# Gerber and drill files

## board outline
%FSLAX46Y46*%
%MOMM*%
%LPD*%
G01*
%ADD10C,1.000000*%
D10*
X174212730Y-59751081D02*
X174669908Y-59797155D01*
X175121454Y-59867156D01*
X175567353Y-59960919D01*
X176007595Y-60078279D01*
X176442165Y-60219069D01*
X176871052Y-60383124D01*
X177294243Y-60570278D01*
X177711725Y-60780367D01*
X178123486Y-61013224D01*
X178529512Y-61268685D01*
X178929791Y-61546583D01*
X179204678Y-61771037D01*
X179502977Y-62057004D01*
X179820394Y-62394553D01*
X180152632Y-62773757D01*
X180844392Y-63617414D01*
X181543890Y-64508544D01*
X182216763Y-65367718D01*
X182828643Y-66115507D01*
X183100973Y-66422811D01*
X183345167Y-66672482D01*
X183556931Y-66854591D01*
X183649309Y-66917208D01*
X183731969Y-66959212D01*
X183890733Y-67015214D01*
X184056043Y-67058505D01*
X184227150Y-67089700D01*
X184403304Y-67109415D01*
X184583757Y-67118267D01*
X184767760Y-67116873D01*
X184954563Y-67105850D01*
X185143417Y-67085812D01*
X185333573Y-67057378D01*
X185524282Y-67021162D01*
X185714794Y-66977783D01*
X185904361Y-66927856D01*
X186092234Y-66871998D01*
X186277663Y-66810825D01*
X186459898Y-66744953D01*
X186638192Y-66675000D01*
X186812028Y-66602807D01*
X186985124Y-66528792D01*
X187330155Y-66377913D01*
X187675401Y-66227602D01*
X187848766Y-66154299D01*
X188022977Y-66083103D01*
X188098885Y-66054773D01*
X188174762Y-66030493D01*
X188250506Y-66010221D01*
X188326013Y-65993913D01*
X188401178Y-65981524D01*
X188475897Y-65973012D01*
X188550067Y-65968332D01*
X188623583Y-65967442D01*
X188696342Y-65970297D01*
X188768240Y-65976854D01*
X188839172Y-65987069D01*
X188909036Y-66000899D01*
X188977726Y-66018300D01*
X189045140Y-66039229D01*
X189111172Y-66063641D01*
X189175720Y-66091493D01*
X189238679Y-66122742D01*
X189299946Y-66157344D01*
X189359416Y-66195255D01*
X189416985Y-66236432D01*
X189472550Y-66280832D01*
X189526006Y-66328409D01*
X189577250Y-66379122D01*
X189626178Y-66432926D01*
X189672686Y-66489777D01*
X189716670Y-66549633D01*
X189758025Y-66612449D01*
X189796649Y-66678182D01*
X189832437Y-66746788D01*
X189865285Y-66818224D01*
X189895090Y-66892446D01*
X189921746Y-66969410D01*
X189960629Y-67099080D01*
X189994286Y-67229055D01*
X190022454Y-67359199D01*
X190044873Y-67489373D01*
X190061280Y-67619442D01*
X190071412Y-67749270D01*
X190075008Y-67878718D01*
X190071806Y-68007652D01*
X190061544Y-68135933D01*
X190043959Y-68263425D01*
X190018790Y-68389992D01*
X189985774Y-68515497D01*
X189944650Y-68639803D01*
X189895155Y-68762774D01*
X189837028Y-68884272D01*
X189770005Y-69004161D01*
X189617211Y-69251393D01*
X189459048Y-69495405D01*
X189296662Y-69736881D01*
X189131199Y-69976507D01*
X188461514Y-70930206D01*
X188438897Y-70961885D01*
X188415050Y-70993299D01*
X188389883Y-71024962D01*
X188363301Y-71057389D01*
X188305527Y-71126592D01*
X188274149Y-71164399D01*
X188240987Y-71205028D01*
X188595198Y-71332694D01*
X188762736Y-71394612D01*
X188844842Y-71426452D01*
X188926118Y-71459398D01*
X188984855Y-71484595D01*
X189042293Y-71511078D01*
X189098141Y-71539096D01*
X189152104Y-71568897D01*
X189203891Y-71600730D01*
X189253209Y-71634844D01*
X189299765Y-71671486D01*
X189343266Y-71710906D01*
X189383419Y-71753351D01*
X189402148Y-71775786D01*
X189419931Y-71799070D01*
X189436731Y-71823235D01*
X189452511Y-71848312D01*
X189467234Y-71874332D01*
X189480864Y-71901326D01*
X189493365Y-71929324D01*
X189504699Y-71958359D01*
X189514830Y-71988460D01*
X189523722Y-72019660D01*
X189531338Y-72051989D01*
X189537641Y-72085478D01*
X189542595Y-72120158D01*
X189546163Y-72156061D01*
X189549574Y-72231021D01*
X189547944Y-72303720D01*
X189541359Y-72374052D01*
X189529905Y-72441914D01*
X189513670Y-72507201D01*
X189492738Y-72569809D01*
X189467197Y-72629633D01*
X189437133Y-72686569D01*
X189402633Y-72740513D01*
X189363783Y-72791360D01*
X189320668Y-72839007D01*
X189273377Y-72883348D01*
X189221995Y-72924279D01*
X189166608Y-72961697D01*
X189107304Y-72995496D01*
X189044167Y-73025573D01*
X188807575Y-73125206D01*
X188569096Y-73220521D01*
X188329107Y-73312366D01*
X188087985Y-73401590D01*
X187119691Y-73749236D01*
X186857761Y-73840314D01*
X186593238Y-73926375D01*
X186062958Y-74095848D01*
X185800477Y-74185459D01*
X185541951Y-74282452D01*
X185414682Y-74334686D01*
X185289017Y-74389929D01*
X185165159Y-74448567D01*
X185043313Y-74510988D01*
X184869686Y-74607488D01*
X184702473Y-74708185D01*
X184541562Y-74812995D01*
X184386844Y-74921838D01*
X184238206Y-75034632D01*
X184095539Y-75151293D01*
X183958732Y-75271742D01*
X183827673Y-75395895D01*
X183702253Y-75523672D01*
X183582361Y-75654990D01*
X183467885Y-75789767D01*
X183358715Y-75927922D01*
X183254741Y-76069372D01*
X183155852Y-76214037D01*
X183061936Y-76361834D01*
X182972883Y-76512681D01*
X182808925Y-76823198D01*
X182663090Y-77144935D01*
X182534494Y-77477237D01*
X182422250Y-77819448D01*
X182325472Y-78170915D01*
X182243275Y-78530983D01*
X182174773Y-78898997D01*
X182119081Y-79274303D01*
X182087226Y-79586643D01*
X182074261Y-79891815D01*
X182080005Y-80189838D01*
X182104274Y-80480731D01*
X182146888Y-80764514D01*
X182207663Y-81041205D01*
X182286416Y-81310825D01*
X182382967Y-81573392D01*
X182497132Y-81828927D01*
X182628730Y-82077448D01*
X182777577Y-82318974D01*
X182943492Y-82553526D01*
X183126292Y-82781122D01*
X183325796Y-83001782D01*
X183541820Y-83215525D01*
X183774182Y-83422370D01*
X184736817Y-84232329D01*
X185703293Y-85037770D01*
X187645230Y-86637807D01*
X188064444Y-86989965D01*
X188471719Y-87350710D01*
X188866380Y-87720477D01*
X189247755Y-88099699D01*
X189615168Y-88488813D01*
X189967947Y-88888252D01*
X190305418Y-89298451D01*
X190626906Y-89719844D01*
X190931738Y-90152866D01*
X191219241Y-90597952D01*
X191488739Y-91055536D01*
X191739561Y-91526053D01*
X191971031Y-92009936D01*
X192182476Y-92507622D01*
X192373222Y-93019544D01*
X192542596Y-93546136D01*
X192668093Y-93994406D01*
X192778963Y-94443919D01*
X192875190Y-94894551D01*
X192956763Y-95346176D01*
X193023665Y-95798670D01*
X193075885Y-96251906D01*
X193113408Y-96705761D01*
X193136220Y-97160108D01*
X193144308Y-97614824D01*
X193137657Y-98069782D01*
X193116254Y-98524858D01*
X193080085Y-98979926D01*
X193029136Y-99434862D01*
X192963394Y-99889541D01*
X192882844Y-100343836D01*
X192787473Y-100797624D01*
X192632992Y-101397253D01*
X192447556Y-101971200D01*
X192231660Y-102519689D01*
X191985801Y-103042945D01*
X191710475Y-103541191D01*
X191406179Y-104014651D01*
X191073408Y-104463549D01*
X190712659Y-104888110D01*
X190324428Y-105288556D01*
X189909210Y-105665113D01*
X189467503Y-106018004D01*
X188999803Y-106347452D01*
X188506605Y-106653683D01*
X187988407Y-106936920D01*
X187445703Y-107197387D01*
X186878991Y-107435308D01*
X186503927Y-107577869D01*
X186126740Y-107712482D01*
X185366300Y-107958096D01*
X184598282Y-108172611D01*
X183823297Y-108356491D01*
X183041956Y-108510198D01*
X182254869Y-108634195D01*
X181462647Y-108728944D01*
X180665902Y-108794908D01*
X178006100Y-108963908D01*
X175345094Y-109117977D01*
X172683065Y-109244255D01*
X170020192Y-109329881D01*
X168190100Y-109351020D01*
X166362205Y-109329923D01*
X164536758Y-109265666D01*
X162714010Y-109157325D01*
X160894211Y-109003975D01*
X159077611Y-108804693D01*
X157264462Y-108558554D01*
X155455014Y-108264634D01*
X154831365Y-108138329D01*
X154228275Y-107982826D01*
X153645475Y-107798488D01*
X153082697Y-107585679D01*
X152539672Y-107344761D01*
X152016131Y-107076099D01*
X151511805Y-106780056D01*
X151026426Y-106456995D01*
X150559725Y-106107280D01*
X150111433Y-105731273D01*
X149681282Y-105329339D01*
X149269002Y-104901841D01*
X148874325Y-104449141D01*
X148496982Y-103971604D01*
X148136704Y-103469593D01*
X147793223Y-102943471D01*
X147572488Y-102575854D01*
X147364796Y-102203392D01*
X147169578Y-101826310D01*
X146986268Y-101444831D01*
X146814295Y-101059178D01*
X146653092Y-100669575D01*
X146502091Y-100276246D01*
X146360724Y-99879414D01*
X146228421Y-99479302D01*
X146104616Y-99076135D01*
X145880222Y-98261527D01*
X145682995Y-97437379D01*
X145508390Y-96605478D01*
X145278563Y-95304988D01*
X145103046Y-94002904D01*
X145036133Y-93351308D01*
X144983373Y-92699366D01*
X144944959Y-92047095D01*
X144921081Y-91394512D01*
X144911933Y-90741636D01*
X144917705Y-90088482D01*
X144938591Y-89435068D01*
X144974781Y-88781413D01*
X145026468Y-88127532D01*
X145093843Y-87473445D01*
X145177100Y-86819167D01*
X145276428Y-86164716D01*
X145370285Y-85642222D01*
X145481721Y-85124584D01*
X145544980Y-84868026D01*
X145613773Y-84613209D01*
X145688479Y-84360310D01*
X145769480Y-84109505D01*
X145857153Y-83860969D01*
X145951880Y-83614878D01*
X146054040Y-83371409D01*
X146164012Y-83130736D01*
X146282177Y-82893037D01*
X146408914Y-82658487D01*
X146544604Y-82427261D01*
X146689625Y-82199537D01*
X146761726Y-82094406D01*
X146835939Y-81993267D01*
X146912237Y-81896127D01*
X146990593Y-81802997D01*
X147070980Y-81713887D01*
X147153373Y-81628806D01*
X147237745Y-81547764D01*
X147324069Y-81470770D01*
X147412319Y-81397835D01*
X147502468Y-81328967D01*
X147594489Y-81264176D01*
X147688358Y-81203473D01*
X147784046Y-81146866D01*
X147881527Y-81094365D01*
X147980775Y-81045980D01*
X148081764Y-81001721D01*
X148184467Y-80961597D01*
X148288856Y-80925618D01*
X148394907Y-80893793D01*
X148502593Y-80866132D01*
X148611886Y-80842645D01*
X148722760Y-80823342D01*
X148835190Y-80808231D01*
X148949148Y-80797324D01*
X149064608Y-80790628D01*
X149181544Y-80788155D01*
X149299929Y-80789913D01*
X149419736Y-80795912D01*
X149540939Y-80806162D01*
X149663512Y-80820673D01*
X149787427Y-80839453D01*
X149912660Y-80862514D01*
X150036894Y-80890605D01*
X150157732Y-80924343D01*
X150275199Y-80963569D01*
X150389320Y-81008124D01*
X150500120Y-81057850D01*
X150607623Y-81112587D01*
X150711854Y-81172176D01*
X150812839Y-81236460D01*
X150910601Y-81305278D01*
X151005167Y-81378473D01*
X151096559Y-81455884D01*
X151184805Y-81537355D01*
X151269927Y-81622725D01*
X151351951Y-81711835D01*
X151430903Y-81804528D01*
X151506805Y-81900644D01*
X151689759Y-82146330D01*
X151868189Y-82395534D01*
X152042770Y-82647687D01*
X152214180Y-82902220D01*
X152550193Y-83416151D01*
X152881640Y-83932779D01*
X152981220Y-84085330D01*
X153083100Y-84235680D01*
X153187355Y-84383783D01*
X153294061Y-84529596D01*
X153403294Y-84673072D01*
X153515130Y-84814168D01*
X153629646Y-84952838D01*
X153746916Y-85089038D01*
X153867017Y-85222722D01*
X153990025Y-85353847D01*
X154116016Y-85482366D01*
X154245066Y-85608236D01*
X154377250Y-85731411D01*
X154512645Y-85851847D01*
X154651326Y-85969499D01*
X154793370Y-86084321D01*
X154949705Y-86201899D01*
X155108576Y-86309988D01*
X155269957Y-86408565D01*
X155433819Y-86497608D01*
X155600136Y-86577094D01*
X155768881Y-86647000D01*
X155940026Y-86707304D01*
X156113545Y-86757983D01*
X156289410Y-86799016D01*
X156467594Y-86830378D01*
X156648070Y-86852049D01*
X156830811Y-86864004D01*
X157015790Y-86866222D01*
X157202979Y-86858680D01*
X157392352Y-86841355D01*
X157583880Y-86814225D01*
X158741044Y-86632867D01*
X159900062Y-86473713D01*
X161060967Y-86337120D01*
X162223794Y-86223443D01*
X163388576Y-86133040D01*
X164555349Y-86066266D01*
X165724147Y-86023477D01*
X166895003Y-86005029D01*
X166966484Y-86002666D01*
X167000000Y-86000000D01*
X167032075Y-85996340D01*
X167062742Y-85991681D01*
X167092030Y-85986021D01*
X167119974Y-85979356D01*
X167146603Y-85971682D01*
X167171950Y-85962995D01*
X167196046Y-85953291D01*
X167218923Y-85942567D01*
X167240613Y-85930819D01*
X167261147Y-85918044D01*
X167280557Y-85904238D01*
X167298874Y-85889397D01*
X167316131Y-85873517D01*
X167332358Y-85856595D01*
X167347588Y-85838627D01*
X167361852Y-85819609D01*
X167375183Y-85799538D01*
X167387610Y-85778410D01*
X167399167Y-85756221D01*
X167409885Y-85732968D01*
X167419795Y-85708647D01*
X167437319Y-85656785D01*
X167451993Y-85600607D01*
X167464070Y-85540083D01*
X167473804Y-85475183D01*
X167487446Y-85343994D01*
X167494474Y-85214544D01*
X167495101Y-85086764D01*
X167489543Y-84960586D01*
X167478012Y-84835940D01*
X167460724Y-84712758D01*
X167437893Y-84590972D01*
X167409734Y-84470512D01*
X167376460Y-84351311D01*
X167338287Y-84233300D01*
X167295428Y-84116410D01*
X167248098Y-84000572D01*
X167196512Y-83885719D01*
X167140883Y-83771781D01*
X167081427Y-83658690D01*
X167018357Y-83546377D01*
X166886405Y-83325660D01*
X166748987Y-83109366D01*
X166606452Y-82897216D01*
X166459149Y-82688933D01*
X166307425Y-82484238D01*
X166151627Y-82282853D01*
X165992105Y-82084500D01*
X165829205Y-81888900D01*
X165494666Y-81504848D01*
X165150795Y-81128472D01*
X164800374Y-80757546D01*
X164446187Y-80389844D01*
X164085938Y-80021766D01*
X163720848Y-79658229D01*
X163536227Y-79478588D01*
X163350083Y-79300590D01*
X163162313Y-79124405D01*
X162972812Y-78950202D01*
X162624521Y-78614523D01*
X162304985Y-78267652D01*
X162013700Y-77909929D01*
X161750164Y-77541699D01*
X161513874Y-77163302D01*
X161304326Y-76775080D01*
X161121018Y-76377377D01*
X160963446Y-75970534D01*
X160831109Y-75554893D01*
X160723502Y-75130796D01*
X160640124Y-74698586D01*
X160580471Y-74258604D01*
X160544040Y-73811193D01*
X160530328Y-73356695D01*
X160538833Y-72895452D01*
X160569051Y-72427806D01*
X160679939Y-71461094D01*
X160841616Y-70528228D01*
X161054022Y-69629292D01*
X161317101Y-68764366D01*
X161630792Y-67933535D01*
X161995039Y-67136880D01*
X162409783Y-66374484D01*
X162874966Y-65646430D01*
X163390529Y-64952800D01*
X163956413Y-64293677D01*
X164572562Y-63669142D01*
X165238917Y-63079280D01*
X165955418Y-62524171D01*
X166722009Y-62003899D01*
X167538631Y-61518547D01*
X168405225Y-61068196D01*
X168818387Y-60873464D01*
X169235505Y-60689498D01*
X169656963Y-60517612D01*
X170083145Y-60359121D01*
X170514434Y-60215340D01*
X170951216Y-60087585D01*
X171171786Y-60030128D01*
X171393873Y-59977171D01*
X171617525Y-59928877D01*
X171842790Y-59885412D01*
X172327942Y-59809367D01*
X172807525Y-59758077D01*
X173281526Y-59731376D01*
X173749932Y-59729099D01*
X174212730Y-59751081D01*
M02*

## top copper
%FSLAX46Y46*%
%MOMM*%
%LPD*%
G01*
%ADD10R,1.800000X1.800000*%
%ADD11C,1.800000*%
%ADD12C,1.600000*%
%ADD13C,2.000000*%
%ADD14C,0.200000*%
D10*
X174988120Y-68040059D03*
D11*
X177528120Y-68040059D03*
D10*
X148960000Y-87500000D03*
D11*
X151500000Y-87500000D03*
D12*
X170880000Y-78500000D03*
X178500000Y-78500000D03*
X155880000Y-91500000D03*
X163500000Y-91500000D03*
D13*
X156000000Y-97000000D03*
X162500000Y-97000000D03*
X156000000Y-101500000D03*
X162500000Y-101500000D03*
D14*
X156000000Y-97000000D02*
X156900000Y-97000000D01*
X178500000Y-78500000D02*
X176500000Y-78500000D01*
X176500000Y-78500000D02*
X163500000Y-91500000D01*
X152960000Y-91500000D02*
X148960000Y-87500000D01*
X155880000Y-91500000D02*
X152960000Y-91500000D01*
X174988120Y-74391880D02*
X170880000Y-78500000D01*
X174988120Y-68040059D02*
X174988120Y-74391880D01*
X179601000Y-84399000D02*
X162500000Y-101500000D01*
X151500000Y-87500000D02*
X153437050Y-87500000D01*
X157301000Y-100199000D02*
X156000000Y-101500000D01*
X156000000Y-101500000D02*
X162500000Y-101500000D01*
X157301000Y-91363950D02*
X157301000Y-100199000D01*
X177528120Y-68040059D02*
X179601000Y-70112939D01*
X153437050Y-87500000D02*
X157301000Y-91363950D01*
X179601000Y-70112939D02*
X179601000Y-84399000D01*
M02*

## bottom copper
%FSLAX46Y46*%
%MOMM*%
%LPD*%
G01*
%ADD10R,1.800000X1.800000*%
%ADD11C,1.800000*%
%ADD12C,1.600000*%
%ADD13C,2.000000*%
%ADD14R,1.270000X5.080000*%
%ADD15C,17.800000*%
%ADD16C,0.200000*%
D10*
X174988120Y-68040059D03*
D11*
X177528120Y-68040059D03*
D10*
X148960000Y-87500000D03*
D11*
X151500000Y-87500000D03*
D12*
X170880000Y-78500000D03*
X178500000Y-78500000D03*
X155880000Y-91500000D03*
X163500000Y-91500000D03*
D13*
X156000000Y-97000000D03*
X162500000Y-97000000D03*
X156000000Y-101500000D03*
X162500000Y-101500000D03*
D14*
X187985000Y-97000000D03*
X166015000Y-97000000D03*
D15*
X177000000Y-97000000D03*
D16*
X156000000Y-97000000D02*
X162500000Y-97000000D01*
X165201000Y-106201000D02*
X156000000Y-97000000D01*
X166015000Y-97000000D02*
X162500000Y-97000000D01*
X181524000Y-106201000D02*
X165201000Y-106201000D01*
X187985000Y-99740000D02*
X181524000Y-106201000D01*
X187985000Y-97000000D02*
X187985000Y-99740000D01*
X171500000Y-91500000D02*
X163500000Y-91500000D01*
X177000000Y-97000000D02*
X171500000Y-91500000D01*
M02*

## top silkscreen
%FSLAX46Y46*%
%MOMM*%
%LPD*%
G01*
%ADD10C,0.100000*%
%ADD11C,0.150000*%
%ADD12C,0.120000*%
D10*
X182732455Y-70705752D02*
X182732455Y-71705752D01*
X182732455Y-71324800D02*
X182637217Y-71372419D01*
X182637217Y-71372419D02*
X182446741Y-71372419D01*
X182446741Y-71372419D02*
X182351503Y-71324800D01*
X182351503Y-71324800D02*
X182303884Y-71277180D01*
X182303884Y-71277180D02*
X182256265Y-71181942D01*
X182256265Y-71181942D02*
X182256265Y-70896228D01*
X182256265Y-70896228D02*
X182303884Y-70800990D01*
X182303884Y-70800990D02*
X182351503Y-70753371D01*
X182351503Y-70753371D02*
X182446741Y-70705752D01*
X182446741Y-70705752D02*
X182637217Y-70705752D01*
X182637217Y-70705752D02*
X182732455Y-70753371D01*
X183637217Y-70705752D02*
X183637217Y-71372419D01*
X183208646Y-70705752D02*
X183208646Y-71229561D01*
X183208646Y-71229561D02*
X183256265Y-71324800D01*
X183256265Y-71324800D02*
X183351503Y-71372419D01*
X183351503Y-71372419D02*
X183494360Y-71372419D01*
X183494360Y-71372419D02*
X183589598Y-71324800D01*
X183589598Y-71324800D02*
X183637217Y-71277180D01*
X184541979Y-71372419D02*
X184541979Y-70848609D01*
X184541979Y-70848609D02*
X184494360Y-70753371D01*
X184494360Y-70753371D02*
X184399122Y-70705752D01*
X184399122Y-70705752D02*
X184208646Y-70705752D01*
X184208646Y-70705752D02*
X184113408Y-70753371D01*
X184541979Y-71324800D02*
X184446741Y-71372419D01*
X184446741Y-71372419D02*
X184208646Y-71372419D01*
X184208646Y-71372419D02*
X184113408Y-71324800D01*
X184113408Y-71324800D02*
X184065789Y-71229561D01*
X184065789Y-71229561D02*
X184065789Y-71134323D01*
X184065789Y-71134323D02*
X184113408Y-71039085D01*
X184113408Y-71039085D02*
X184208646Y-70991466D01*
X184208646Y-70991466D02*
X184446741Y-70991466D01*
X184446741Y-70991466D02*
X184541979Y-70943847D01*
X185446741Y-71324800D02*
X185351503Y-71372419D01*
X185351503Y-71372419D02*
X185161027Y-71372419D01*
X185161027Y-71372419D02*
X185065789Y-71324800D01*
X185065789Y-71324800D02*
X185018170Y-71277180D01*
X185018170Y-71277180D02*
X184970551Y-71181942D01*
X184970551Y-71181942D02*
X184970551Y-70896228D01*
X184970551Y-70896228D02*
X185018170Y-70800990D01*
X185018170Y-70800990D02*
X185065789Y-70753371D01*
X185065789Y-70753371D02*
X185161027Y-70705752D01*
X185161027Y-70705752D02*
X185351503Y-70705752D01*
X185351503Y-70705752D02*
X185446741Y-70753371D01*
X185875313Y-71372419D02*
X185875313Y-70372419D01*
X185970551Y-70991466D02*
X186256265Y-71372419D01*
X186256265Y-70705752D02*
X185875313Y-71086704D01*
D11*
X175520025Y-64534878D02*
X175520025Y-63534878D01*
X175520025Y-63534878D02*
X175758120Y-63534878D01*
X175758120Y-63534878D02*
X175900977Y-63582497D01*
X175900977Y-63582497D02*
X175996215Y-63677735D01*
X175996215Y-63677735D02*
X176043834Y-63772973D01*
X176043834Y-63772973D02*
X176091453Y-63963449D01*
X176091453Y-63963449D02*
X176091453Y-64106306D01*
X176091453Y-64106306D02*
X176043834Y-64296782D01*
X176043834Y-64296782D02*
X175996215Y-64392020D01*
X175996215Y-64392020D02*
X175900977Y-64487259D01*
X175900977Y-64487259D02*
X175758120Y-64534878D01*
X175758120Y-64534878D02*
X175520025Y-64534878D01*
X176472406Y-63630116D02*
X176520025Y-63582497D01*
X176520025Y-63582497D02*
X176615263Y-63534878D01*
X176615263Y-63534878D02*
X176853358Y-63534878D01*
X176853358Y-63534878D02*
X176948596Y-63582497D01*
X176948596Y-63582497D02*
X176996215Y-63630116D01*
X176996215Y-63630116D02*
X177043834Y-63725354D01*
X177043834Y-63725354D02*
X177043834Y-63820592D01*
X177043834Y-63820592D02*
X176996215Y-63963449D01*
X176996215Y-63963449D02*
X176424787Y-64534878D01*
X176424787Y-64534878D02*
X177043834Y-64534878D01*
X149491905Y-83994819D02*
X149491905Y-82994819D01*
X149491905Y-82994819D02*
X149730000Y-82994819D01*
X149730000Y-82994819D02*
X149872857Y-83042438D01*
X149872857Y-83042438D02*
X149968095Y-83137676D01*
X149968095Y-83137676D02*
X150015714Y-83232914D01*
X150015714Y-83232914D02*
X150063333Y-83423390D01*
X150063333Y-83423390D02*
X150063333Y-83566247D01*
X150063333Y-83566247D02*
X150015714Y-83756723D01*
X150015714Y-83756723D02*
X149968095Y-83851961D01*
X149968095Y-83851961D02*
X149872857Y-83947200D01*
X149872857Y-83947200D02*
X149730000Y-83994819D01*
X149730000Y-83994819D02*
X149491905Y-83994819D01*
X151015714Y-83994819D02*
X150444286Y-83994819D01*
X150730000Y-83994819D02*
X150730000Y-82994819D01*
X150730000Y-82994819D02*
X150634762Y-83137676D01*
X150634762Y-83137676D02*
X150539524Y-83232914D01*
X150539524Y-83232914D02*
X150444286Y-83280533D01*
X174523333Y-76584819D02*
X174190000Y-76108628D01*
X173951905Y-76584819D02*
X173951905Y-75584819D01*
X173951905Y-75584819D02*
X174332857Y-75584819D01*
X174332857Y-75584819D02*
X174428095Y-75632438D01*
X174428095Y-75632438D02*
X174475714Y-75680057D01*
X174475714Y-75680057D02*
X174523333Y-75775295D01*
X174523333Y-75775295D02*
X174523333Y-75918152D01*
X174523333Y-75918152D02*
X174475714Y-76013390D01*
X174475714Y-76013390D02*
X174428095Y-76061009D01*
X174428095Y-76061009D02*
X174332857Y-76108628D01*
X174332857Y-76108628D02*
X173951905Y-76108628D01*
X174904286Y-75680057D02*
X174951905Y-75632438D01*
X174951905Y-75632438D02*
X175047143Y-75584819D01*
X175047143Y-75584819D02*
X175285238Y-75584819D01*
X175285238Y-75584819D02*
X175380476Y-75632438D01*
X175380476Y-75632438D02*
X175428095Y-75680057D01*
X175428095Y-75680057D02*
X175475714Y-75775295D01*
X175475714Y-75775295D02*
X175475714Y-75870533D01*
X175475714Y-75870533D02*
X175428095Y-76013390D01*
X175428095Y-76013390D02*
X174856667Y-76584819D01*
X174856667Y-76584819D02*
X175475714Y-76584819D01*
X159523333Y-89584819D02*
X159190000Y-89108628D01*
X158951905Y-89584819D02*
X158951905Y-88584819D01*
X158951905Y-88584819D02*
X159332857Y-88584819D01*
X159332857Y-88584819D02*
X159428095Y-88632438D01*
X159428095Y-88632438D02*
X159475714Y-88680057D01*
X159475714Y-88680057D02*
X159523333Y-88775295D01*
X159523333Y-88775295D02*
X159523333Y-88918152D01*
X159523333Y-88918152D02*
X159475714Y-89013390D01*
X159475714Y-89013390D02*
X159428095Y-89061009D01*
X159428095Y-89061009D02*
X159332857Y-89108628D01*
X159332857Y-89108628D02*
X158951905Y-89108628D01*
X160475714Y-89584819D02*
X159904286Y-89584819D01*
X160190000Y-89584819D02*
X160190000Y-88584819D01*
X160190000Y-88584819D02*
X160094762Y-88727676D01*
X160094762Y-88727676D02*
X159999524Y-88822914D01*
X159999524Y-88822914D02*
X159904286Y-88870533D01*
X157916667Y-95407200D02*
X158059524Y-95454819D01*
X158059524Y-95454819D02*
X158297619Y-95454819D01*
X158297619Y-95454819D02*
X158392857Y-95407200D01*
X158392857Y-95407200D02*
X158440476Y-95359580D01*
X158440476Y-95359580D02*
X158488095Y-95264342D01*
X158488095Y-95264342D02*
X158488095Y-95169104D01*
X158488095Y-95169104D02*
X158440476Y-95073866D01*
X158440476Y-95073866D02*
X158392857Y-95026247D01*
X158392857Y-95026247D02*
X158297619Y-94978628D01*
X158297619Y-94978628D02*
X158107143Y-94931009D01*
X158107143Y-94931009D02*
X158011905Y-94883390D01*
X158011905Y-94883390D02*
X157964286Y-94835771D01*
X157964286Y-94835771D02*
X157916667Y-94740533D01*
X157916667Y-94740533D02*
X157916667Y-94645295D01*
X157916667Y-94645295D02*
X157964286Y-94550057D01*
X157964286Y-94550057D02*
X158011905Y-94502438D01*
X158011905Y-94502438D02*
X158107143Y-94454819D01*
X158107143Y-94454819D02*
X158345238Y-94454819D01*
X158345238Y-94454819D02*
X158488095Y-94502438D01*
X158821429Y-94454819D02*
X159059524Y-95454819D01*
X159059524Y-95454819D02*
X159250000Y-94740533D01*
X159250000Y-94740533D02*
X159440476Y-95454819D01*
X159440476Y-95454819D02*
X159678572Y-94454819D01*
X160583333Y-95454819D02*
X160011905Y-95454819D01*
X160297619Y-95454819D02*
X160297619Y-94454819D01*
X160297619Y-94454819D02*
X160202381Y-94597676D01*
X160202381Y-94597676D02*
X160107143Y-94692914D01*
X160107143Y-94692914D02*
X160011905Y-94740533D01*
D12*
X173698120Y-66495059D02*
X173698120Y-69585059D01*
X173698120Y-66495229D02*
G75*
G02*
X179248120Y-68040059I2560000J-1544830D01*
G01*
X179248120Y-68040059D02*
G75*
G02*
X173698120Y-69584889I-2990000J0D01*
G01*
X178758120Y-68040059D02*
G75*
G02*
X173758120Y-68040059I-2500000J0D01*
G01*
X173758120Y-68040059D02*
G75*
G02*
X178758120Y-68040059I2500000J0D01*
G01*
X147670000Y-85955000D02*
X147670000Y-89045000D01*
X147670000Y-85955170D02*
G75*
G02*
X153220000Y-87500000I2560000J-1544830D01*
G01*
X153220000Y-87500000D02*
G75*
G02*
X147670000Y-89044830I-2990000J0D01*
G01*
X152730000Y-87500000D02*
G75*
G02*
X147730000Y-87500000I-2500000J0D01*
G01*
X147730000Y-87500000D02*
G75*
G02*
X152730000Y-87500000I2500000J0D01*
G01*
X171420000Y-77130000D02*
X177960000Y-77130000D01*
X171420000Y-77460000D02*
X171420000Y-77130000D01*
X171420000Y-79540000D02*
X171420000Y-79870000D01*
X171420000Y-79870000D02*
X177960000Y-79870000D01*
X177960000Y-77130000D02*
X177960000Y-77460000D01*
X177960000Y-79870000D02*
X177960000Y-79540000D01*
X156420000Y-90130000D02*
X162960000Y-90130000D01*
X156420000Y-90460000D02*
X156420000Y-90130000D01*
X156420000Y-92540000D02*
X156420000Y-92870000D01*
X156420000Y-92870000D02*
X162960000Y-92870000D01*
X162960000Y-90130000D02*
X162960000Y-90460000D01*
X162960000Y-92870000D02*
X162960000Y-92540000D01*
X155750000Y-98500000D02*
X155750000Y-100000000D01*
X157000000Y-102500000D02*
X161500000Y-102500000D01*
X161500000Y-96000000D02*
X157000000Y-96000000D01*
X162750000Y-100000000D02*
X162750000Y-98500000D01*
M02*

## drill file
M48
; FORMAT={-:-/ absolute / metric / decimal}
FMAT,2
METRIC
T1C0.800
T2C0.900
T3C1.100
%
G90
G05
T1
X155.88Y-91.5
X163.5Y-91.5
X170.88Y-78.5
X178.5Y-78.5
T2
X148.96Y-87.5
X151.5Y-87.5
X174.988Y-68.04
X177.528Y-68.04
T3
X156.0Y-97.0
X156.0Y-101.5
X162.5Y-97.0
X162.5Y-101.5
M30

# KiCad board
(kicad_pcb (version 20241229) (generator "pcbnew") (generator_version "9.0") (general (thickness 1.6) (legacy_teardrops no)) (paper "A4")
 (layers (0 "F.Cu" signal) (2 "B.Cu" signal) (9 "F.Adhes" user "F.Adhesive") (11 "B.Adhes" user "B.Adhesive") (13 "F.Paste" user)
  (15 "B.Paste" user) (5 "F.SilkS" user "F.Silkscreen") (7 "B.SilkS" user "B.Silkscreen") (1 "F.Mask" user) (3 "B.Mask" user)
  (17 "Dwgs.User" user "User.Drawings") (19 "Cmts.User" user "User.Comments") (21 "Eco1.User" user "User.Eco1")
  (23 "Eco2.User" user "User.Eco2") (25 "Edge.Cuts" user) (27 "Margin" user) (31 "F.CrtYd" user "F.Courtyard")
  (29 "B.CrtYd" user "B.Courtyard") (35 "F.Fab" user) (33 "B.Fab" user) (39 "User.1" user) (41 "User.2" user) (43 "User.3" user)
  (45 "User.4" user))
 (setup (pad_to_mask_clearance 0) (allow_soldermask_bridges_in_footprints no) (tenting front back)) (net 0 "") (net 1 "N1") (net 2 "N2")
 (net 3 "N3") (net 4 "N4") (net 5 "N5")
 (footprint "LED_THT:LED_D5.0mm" (layer "F.Cu") (at 174.98812 68.040059)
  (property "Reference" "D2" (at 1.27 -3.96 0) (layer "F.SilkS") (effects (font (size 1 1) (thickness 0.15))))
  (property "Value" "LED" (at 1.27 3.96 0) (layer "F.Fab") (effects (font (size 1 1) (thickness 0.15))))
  (fp_line (start -1.29 -1.545) (end -1.29 1.545) (stroke (width 0.12) (type solid)) (layer "F.SilkS"))
  (fp_arc (start -1.29 -1.54483) (mid 2.071779 -2.880495) (end 4.26 0) (stroke (width 0.12) (type solid)) (layer "F.SilkS"))
  (fp_arc (start 4.26 0) (mid 2.071779 2.880495) (end -1.29 1.54483) (stroke (width 0.12) (type solid)) (layer "F.SilkS"))
  (fp_circle (center 1.27 0) (end 3.77 0) (stroke (width 0.12) (type solid)) (fill no) (layer "F.SilkS"))
  (pad "1" thru_hole rect (at 0 0) (size 1.8 1.8) (drill 0.9) (layers "*.Cu" "*.Mask") (remove_unused_layers no) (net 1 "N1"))
  (pad "2" thru_hole circle (at 2.54 0) (size 1.8 1.8) (drill 0.9) (layers "*.Cu" "*.Mask") (remove_unused_layers no) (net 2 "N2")))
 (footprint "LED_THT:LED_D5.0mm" (layer "F.Cu") (at 148.96 87.5)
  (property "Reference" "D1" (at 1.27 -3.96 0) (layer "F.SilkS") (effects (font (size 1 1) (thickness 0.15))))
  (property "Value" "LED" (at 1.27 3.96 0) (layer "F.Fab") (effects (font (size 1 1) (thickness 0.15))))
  (fp_line (start -1.29 -1.545) (end -1.29 1.545) (stroke (width 0.12) (type solid)) (layer "F.SilkS"))
  (fp_arc (start -1.29 -1.54483) (mid 2.071779 -2.880495) (end 4.26 0) (stroke (width 0.12) (type solid)) (layer "F.SilkS"))
  (fp_arc (start 4.26 0) (mid 2.071779 2.880495) (end -1.29 1.54483) (stroke (width 0.12) (type solid)) (layer "F.SilkS"))
  (fp_circle (center 1.27 0) (end 3.77 0) (stroke (width 0.12) (type solid)) (fill no) (layer "F.SilkS"))
  (pad "1" thru_hole rect (at 0 0) (size 1.8 1.8) (drill 0.9) (layers "*.Cu" "*.Mask") (remove_unused_layers no) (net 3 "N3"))
  (pad "2" thru_hole circle (at 2.54 0) (size 1.8 1.8) (drill 0.9) (layers "*.Cu" "*.Mask") (remove_unused_layers no) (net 2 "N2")))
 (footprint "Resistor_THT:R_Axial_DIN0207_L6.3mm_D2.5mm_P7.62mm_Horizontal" (layer "F.Cu") (at 170.88 78.5)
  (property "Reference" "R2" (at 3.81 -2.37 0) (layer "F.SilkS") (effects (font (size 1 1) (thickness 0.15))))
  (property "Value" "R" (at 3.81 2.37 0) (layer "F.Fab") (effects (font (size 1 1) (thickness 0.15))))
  (fp_line (start 0.54 -1.37) (end 7.08 -1.37) (stroke (width 0.12) (type solid)) (layer "F.SilkS"))
  (fp_line (start 0.54 -1.04) (end 0.54 -1.37) (stroke (width 0.12) (type solid)) (layer "F.SilkS"))
  (fp_line (start 0.54 1.04) (end 0.54 1.37) (stroke (width 0.12) (type solid)) (layer "F.SilkS"))
  (fp_line (start 0.54 1.37) (end 7.08 1.37) (stroke (width 0.12) (type solid)) (layer "F.SilkS"))
  (fp_line (start 7.08 -1.37) (end 7.08 -1.04) (stroke (width 0.12) (type solid)) (layer "F.SilkS"))
  (fp_line (start 7.08 1.37) (end 7.08 1.04) (stroke (width 0.12) (type solid)) (layer "F.SilkS"))
  (pad "1" thru_hole circle (at 0 0) (size 1.6 1.6) (drill 0.8) (layers "*.Cu" "*.Mask") (remove_unused_layers no) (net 1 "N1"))
  (pad "2" thru_hole circle (at 7.62 0) (size 1.6 1.6) (drill 0.8) (layers "*.Cu" "*.Mask") (remove_unused_layers no) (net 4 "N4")))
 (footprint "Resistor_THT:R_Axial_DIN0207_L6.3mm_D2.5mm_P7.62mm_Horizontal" (layer "F.Cu") (at 155.88 91.5)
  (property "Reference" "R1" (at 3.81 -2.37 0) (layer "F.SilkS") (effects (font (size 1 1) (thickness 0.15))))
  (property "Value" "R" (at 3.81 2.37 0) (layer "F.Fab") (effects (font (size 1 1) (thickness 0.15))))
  (fp_line (start 0.54 -1.37) (end 7.08 -1.37) (stroke (width 0.12) (type solid)) (layer "F.SilkS"))
  (fp_line (start 0.54 -1.04) (end 0.54 -1.37) (stroke (width 0.12) (type solid)) (layer "F.SilkS"))
  (fp_line (start 0.54 1.04) (end 0.54 1.37) (stroke (width 0.12) (type solid)) (layer "F.SilkS"))
  (fp_line (start 0.54 1.37) (end 7.08 1.37) (stroke (width 0.12) (type solid)) (layer "F.SilkS"))
  (fp_line (start 7.08 -1.37) (end 7.08 -1.04) (stroke (width 0.12) (type solid)) (layer "F.SilkS"))
  (fp_line (start 7.08 1.37) (end 7.08 1.04) (stroke (width 0.12) (type solid)) (layer "F.SilkS"))
  (pad "1" thru_hole circle (at 0 0) (size 1.6 1.6) (drill 0.8) (layers "*.Cu" "*.Mask") (remove_unused_layers no) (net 3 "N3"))
  (pad "2" thru_hole circle (at 7.62 0) (size 1.6 1.6) (drill 0.8) (layers "*.Cu" "*.Mask") (remove_unused_layers no) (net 4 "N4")))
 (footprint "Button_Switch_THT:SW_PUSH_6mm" (layer "F.Cu") (at 156 97)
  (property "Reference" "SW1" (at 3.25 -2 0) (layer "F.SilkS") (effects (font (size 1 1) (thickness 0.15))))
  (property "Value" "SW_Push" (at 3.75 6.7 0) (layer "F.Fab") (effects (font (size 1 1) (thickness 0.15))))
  (fp_line (start -0.25 1.5) (end -0.25 3) (stroke (width 0.12) (type solid)) (layer "F.SilkS"))
  (fp_line (start 1 5.5) (end 5.5 5.5) (stroke (width 0.12) (type solid)) (layer "F.SilkS"))
  (fp_line (start 5.5 -1) (end 1 -1) (stroke (width 0.12) (type solid)) (layer "F.SilkS"))
  (fp_line (start 6.75 3) (end 6.75 1.5) (stroke (width 0.12) (type solid)) (layer "F.SilkS"))
  (pad "1" thru_hole circle (at 0 0 90) (size 2 2) (drill 1.1) (layers "*.Cu" "*.Mask") (remove_unused_layers no) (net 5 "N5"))
  (pad "1" thru_hole circle (at 6.5 0 90) (size 2 2) (drill 1.1) (layers "*.Cu" "*.Mask") (remove_unused_layers no) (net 5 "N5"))
  (pad "2" thru_hole circle (at 0 4.5 90) (size 2 2) (drill 1.1) (layers "*.Cu" "*.Mask") (remove_unused_layers no) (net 2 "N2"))
  (pad "2" thru_hole circle (at 6.5 4.5 90) (size 2 2) (drill 1.1) (layers "*.Cu" "*.Mask") (remove_unused_layers no) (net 2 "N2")))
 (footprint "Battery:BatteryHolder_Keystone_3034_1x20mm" (layer "B.Cu") (at 177 97 180)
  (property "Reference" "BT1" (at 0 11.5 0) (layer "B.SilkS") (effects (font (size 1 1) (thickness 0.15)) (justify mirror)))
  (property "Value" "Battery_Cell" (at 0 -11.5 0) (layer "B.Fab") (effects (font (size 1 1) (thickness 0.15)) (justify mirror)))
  (pad "1" smd rect (at -10.985 0 180) (size 1.27 5.08) (layers "B.Cu" "B.Mask" "B.Paste") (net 5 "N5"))
  (pad "1" smd rect (at 10.985 0 180) (size 1.27 5.08) (layers "B.Cu" "B.Mask" "B.Paste") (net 5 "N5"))
  (pad "2" smd circle (at 0 0 180) (size 17.8 17.8) (layers "B.Cu" "B.Mask") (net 4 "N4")))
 (gr_poly
  (pts (xy 174.21273 59.751081) (xy 174.669908 59.797155) (xy 175.121454 59.867156) (xy 175.567353 59.960919) (xy 176.007595 60.078279)
   (xy 176.442165 60.219069) (xy 176.871052 60.383124) (xy 177.294243 60.570278) (xy 177.711725 60.780367) (xy 178.123486 61.013224)
   (xy 178.529512 61.268685) (xy 178.929791 61.546583) (xy 179.204678 61.771037) (xy 179.502977 62.057004) (xy 179.820394 62.394553)
   (xy 180.152632 62.773757) (xy 180.844392 63.617414) (xy 181.54389 64.508544) (xy 182.216763 65.367718) (xy 182.828643 66.115507)
   (xy 183.100973 66.422811) (xy 183.345167 66.672482) (xy 183.556931 66.854591) (xy 183.649309 66.917208) (xy 183.731969 66.959212)
   (xy 183.890733 67.015214) (xy 184.056043 67.058505) (xy 184.22715 67.0897) (xy 184.403304 67.109415) (xy 184.583757 67.118267)
   (xy 184.76776 67.116873) (xy 184.954563 67.10585) (xy 185.143417 67.085812) (xy 185.333573 67.057378) (xy 185.524282 67.021162)
   (xy 185.714794 66.977783) (xy 185.904361 66.927856) (xy 186.092234 66.871998) (xy 186.277663 66.810825) (xy 186.459898 66.744953)
   (xy 186.638192 66.675) (xy 186.812028 66.602807) (xy 186.985124 66.528792) (xy 187.330155 66.377913) (xy 187.675401 66.227602)
   (xy 187.848766 66.154299) (xy 188.022977 66.083103) (xy 188.098885 66.054773) (xy 188.174762 66.030493) (xy 188.250506 66.010221)
   (xy 188.326013 65.993913) (xy 188.401178 65.981524) (xy 188.475897 65.973012) (xy 188.550067 65.968332) (xy 188.623583 65.967442)
   (xy 188.696342 65.970297) (xy 188.76824 65.976854) (xy 188.839172 65.987069) (xy 188.909036 66.000899) (xy 188.977726 66.0183)
   (xy 189.04514 66.039229) (xy 189.111172 66.063641) (xy 189.17572 66.091493) (xy 189.238679 66.122742) (xy 189.299946 66.157344)
   (xy 189.359416 66.195255) (xy 189.416985 66.236432) (xy 189.47255 66.280832) (xy 189.526006 66.328409) (xy 189.57725 66.379122)
   (xy 189.626178 66.432926) (xy 189.672686 66.489777) (xy 189.71667 66.549633) (xy 189.758025 66.612449) (xy 189.796649 66.678182)
   (xy 189.832437 66.746788) (xy 189.865285 66.818224) (xy 189.89509 66.892446) (xy 189.921746 66.96941) (xy 189.960629 67.09908)
   (xy 189.994286 67.229055) (xy 190.022454 67.359199) (xy 190.044873 67.489373) (xy 190.06128 67.619442) (xy 190.071412 67.74927)
   (xy 190.075008 67.878718) (xy 190.071806 68.007652) (xy 190.061544 68.135933) (xy 190.043959 68.263425) (xy 190.01879 68.389992)
   (xy 189.985774 68.515497) (xy 189.94465 68.639803) (xy 189.895155 68.762774) (xy 189.837028 68.884272) (xy 189.770005 69.004161)
   (xy 189.617211 69.251393) (xy 189.459048 69.495405) (xy 189.296662 69.736881) (xy 189.131199 69.976507) (xy 188.461514 70.930206)
   (xy 188.438897 70.961885) (xy 188.41505 70.993299) (xy 188.389883 71.024962) (xy 188.363301 71.057389) (xy 188.305527 71.126592)
   (xy 188.274149 71.164399) (xy 188.240987 71.205028) (xy 188.595198 71.332694) (xy 188.762736 71.394612) (xy 188.844842 71.426452)
   (xy 188.926118 71.459398) (xy 188.984855 71.484595) (xy 189.042293 71.511078) (xy 189.098141 71.539096) (xy 189.152104 71.568897)
   (xy 189.203891 71.60073) (xy 189.253209 71.634844) (xy 189.299765 71.671486) (xy 189.343266 71.710906) (xy 189.383419 71.753351)
   (xy 189.402148 71.775786) (xy 189.419931 71.79907) (xy 189.436731 71.823235) (xy 189.452511 71.848312) (xy 189.467234 71.874332)
   (xy 189.480864 71.901326) (xy 189.493365 71.929324) (xy 189.504699 71.958359) (xy 189.51483 71.98846) (xy 189.523722 72.01966)
   (xy 189.531338 72.051989) (xy 189.537641 72.085478) (xy 189.542595 72.120158) (xy 189.546163 72.156061) (xy 189.549574 72.231021)
   (xy 189.547944 72.30372) (xy 189.541359 72.374052) (xy 189.529905 72.441914) (xy 189.51367 72.507201) (xy 189.492738 72.569809)
   (xy 189.467197 72.629633) (xy 189.437133 72.686569) (xy 189.402633 72.740513) (xy 189.363783 72.79136) (xy 189.320668 72.839007)
   (xy 189.273377 72.883348) (xy 189.221995 72.924279) (xy 189.166608 72.961697) (xy 189.107304 72.995496) (xy 189.044167 73.025573)
   (xy 188.807575 73.125206) (xy 188.569096 73.220521) (xy 188.329107 73.312366) (xy 188.087985 73.40159) (xy 187.119691 73.749236)
   (xy 186.857761 73.840314) (xy 186.593238 73.926375) (xy 186.062958 74.095848) (xy 185.800477 74.185459) (xy 185.541951 74.282452)
   (xy 185.414682 74.334686) (xy 185.289017 74.389929) (xy 185.165159 74.448567) (xy 185.043313 74.510988) (xy 184.869686 74.607488)
   (xy 184.702473 74.708185) (xy 184.541562 74.812995) (xy 184.386844 74.921838) (xy 184.238206 75.034632) (xy 184.095539 75.151293)
   (xy 183.958732 75.271742) (xy 183.827673 75.395895) (xy 183.702253 75.523672) (xy 183.582361 75.65499) (xy 183.467885 75.789767)
   (xy 183.358715 75.927922) (xy 183.254741 76.069372) (xy 183.155852 76.214037) (xy 183.061936 76.361834) (xy 182.972883 76.512681)
   (xy 182.808925 76.823198) (xy 182.66309 77.144935) (xy 182.534494 77.477237) (xy 182.42225 77.819448) (xy 182.325472 78.170915)
   (xy 182.243275 78.530983) (xy 182.174773 78.898997) (xy 182.119081 79.274303) (xy 182.087226 79.586643) (xy 182.074261 79.891815)
   (xy 182.080005 80.189838) (xy 182.104274 80.480731) (xy 182.146888 80.764514) (xy 182.207663 81.041205) (xy 182.286416 81.310825)
   (xy 182.382967 81.573392) (xy 182.497132 81.828927) (xy 182.62873 82.077448) (xy 182.777577 82.318974) (xy 182.943492 82.553526)
   (xy 183.126292 82.781122) (xy 183.325796 83.001782) (xy 183.54182 83.215525) (xy 183.774182 83.42237) (xy 184.736817 84.232329)
   (xy 185.703293 85.03777) (xy 187.64523 86.637807) (xy 188.064444 86.989965) (xy 188.471719 87.35071) (xy 188.86638 87.720477)
   (xy 189.247755 88.099699) (xy 189.615168 88.488813) (xy 189.967947 88.888252) (xy 190.305418 89.298451) (xy 190.626906 89.719844)
   (xy 190.931738 90.152866) (xy 191.219241 90.597952) (xy 191.488739 91.055536) (xy 191.739561 91.526053) (xy 191.971031 92.009936)
   (xy 192.182476 92.507622) (xy 192.373222 93.019544) (xy 192.542596 93.546136) (xy 192.668093 93.994406) (xy 192.778963 94.443919)
   (xy 192.87519 94.894551) (xy 192.956763 95.346176) (xy 193.023665 95.79867) (xy 193.075885 96.251906) (xy 193.113408 96.705761)
   (xy 193.13622 97.160108) (xy 193.144308 97.614824) (xy 193.137657 98.069782) (xy 193.116254 98.524858) (xy 193.080085 98.979926)
   (xy 193.029136 99.434862) (xy 192.963394 99.889541) (xy 192.882844 100.343836) (xy 192.787473 100.797624) (xy 192.632992 101.397253)
   (xy 192.447556 101.9712) (xy 192.23166 102.519689) (xy 191.985801 103.042945) (xy 191.710475 103.541191) (xy 191.406179 104.014651)
   (xy 191.073408 104.463549) (xy 190.712659 104.88811) (xy 190.324428 105.288556) (xy 189.90921 105.665113) (xy 189.467503 106.018004)
   (xy 188.999803 106.347452) (xy 188.506605 106.653683) (xy 187.988407 106.93692) (xy 187.445703 107.197387) (xy 186.878991 107.435308)
   (xy 186.503927 107.577869) (xy 186.12674 107.712482) (xy 185.3663 107.958096) (xy 184.598282 108.172611) (xy 183.823297 108.356491)
   (xy 183.041956 108.510198) (xy 182.254869 108.634195) (xy 181.462647 108.728944) (xy 180.665902 108.794908) (xy 178.0061 108.963908)
   (xy 175.345094 109.117977) (xy 172.683065 109.244255) (xy 170.020192 109.329881) (xy 168.1901 109.35102) (xy 166.362205 109.329923)
   (xy 164.536758 109.265666) (xy 162.71401 109.157325) (xy 160.894211 109.003975) (xy 159.077611 108.804693) (xy 157.264462 108.558554)
   (xy 155.455014 108.264634) (xy 154.831365 108.138329) (xy 154.228275 107.982826) (xy 153.645475 107.798488) (xy 153.082697 107.585679)
   (xy 152.539672 107.344761) (xy 152.016131 107.076099) (xy 151.511805 106.780056) (xy 151.026426 106.456995) (xy 150.559725 106.10728)
   (xy 150.111433 105.731273) (xy 149.681282 105.329339) (xy 149.269002 104.901841) (xy 148.874325 104.449141) (xy 148.496982 103.971604)
   (xy 148.136704 103.469593) (xy 147.793223 102.943471) (xy 147.572488 102.575854) (xy 147.364796 102.203392) (xy 147.169578 101.82631)
   (xy 146.986268 101.444831) (xy 146.814295 101.059178) (xy 146.653092 100.669575) (xy 146.502091 100.276246) (xy 146.360724 99.879414)
   (xy 146.228421 99.479302) (xy 146.104616 99.076135) (xy 145.880222 98.261527) (xy 145.682995 97.437379) (xy 145.50839 96.605478)
   (xy 145.278563 95.304988) (xy 145.103046 94.002904) (xy 145.036133 93.351308) (xy 144.983373 92.699366) (xy 144.944959 92.047095)
   (xy 144.921081 91.394512) (xy 144.911933 90.741636) (xy 144.917705 90.088482) (xy 144.938591 89.435068) (xy 144.974781 88.781413)
   (xy 145.026468 88.127532) (xy 145.093843 87.473445) (xy 145.1771 86.819167) (xy 145.276428 86.164716) (xy 145.370285 85.642222)
   (xy 145.481721 85.124584) (xy 145.54498 84.868026) (xy 145.613773 84.613209) (xy 145.688479 84.36031) (xy 145.76948 84.109505)
   (xy 145.857153 83.860969) (xy 145.95188 83.614878) (xy 146.05404 83.371409) (xy 146.164012 83.130736) (xy 146.282177 82.893037)
   (xy 146.408914 82.658487) (xy 146.544604 82.427261) (xy 146.689625 82.199537) (xy 146.761726 82.094406) (xy 146.835939 81.993267)
   (xy 146.912237 81.896127) (xy 146.990593 81.802997) (xy 147.07098 81.713887) (xy 147.153373 81.628806) (xy 147.237745 81.547764)
   (xy 147.324069 81.47077) (xy 147.412319 81.397835) (xy 147.502468 81.328967) (xy 147.594489 81.264176) (xy 147.688358 81.203473)
   (xy 147.784046 81.146866) (xy 147.881527 81.094365) (xy 147.980775 81.04598) (xy 148.081764 81.001721) (xy 148.184467 80.961597)
   (xy 148.288856 80.925618) (xy 148.394907 80.893793) (xy 148.502593 80.866132) (xy 148.611886 80.842645) (xy 148.72276 80.823342)
   (xy 148.83519 80.808231) (xy 148.949148 80.797324) (xy 149.064608 80.790628) (xy 149.181544 80.788155) (xy 149.299929 80.789913)
   (xy 149.419736 80.795912) (xy 149.540939 80.806162) (xy 149.663512 80.820673) (xy 149.787427 80.839453) (xy 149.91266 80.862514)
   (xy 150.036894 80.890605) (xy 150.157732 80.924343) (xy 150.275199 80.963569) (xy 150.38932 81.008124) (xy 150.50012 81.05785)
   (xy 150.607623 81.112587) (xy 150.711854 81.172176) (xy 150.812839 81.23646) (xy 150.910601 81.305278) (xy 151.005167 81.378473)
   (xy 151.096559 81.455884) (xy 151.184805 81.537355) (xy 151.269927 81.622725) (xy 151.351951 81.711835) (xy 151.430903 81.804528)
   (xy 151.506805 81.900644) (xy 151.689759 82.14633) (xy 151.868189 82.395534) (xy 152.04277 82.647687) (xy 152.21418 82.90222)
   (xy 152.550193 83.416151) (xy 152.88164 83.932779) (xy 152.98122 84.08533) (xy 153.0831 84.23568) (xy 153.187355 84.383783)
   (xy 153.294061 84.529596) (xy 153.403294 84.673072) (xy 153.51513 84.814168) (xy 153.629646 84.952838) (xy 153.746916 85.089038)
   (xy 153.867017 85.222722) (xy 153.990025 85.353847) (xy 154.116016 85.482366) (xy 154.245066 85.608236) (xy 154.37725 85.731411)
   (xy 154.512645 85.851847) (xy 154.651326 85.969499) (xy 154.79337 86.084321) (xy 154.949705 86.201899) (xy 155.108576 86.309988)
   (xy 155.269957 86.408565) (xy 155.433819 86.497608) (xy 155.600136 86.577094) (xy 155.768881 86.647) (xy 155.940026 86.707304)
   (xy 156.113545 86.757983) (xy 156.28941 86.799016) (xy 156.467594 86.830378) (xy 156.64807 86.852049) (xy 156.830811 86.864004)
   (xy 157.01579 86.866222) (xy 157.202979 86.85868) (xy 157.392352 86.841355) (xy 157.58388 86.814225) (xy 158.741044 86.632867)
   (xy 159.900062 86.473713) (xy 161.060967 86.33712) (xy 162.223794 86.223443) (xy 163.388576 86.13304) (xy 164.555349 86.066266)
   (xy 165.724147 86.023477) (xy 166.895003 86.005029) (xy 166.966484 86.002666) (xy 167 86) (xy 167.032075 85.99634)
   (xy 167.062742 85.991681) (xy 167.09203 85.986021) (xy 167.119974 85.979356) (xy 167.146603 85.971682) (xy 167.17195 85.962995)
   (xy 167.196046 85.953291) (xy 167.218923 85.942567) (xy 167.240613 85.930819) (xy 167.261147 85.918044) (xy 167.280557 85.904238)
   (xy 167.298874 85.889397) (xy 167.316131 85.873517) (xy 167.332358 85.856595) (xy 167.347588 85.838627) (xy 167.361852 85.819609)
   (xy 167.375183 85.799538) (xy 167.38761 85.77841) (xy 167.399167 85.756221) (xy 167.409885 85.732968) (xy 167.419795 85.708647)
   (xy 167.437319 85.656785) (xy 167.451993 85.600607) (xy 167.46407 85.540083) (xy 167.473804 85.475183) (xy 167.487446 85.343994)
   (xy 167.494474 85.214544) (xy 167.495101 85.086764) (xy 167.489543 84.960586) (xy 167.478012 84.83594) (xy 167.460724 84.712758)
   (xy 167.437893 84.590972) (xy 167.409734 84.470512) (xy 167.37646 84.351311) (xy 167.338287 84.2333) (xy 167.295428 84.11641)
   (xy 167.248098 84.000572) (xy 167.196512 83.885719) (xy 167.140883 83.771781) (xy 167.081427 83.65869) (xy 167.018357 83.546377)
   (xy 166.886405 83.32566) (xy 166.748987 83.109366) (xy 166.606452 82.897216) (xy 166.459149 82.688933) (xy 166.307425 82.484238)
   (xy 166.151627 82.282853) (xy 165.992105 82.0845) (xy 165.829205 81.8889) (xy 165.494666 81.504848) (xy 165.150795 81.128472)
   (xy 164.800374 80.757546) (xy 164.446187 80.389844) (xy 164.085938 80.021766) (xy 163.720848 79.658229) (xy 163.536227 79.478588)
   (xy 163.350083 79.30059) (xy 163.162313 79.124405) (xy 162.972812 78.950202) (xy 162.624521 78.614523) (xy 162.304985 78.267652)
   (xy 162.0137 77.909929) (xy 161.750164 77.541699) (xy 161.513874 77.163302) (xy 161.304326 76.77508) (xy 161.121018 76.377377)
   (xy 160.963446 75.970534) (xy 160.831109 75.554893) (xy 160.723502 75.130796) (xy 160.640124 74.698586) (xy 160.580471 74.258604)
   (xy 160.54404 73.811193) (xy 160.530328 73.356695) (xy 160.538833 72.895452) (xy 160.569051 72.427806) (xy 160.679939 71.461094)
   (xy 160.841616 70.528228) (xy 161.054022 69.629292) (xy 161.317101 68.764366) (xy 161.630792 67.933535) (xy 161.995039 67.13688)
   (xy 162.409783 66.374484) (xy 162.874966 65.64643) (xy 163.390529 64.9528) (xy 163.956413 64.293677) (xy 164.572562 63.669142)
   (xy 165.238917 63.07928) (xy 165.955418 62.524171) (xy 166.722009 62.003899) (xy 167.538631 61.518547) (xy 168.405225 61.068196)
   (xy 168.818387 60.873464) (xy 169.235505 60.689498) (xy 169.656963 60.517612) (xy 170.083145 60.359121) (xy 170.514434 60.21534)
   (xy 170.951216 60.087585) (xy 171.171786 60.030128) (xy 171.393873 59.977171) (xy 171.617525 59.928877) (xy 171.84279 59.885412)
   (xy 172.327942 59.809367) (xy 172.807525 59.758077) (xy 173.281526 59.731376) (xy 173.749932 59.729099))
  (stroke (width 1) (type solid)) (fill no) (layer "Edge.Cuts"))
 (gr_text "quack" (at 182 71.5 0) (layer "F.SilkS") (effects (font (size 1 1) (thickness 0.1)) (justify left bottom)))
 (segment (start 156 97) (end 156.9 97) (width 0.2) (layer "F.Cu") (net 5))
 (segment (start 156 97) (end 162.5 97) (width 0.2) (layer "B.Cu") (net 5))
 (segment (start 165.201 106.201) (end 156 97) (width 0.2) (layer "B.Cu") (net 5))
 (segment (start 166.015 97) (end 162.5 97) (width 0.2) (layer "B.Cu") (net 5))
 (segment (start 181.524 106.201) (end 165.201 106.201) (width 0.2) (layer "B.Cu") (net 5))
 (segment (start 187.985 99.74) (end 181.524 106.201) (width 0.2) (layer "B.Cu") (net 5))
 (segment (start 187.985 97) (end 187.985 99.74) (width 0.2) (layer "B.Cu") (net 5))
 (segment (start 178.5 78.5) (end 176.5 78.5) (width 0.2) (layer "F.Cu") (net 4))
 (segment (start 176.5 78.5) (end 163.5 91.5) (width 0.2) (layer "F.Cu") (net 4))
 (segment (start 171.5 91.5) (end 163.5 91.5) (width 0.2) (layer "B.Cu") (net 4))
 (segment (start 177 97) (end 171.5 91.5) (width 0.2) (layer "B.Cu") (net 4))
 (segment (start 152.96 91.5) (end 148.96 87.5) (width 0.2) (layer "F.Cu") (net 3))
 (segment (start 155.88 91.5) (end 152.96 91.5) (width 0.2) (layer "F.Cu") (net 3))
 (segment (start 174.98812 74.39188) (end 170.88 78.5) (width 0.2) (layer "F.Cu") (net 1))
 (segment (start 174.98812 68.040059) (end 174.98812 74.39188) (width 0.2) (layer "F.Cu") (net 1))
 (segment (start 179.601 84.399) (end 162.5 101.5) (width 0.2) (layer "F.Cu") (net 2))
 (segment (start 151.5 87.5) (end 153.43705 87.5) (width 0.2) (layer "F.Cu") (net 2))
 (segment (start 157.301 100.199) (end 156 101.5) (width 0.2) (layer "F.Cu") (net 2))
 (segment (start 156 101.5) (end 162.5 101.5) (width 0.2) (layer "F.Cu") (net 2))
 (segment (start 157.301 91.36395) (end 157.301 100.199) (width 0.2) (layer "F.Cu") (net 2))
 (segment (start 177.52812 68.040059) (end 179.601 70.112939) (width 0.2) (layer "F.Cu") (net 2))
 (segment (start 153.43705 87.5) (end 157.301 91.36395) (width 0.2) (layer "F.Cu") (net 2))
 (segment (start 179.601 70.112939) (end 179.601 84.399) (width 0.2) (layer "F.Cu") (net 2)))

